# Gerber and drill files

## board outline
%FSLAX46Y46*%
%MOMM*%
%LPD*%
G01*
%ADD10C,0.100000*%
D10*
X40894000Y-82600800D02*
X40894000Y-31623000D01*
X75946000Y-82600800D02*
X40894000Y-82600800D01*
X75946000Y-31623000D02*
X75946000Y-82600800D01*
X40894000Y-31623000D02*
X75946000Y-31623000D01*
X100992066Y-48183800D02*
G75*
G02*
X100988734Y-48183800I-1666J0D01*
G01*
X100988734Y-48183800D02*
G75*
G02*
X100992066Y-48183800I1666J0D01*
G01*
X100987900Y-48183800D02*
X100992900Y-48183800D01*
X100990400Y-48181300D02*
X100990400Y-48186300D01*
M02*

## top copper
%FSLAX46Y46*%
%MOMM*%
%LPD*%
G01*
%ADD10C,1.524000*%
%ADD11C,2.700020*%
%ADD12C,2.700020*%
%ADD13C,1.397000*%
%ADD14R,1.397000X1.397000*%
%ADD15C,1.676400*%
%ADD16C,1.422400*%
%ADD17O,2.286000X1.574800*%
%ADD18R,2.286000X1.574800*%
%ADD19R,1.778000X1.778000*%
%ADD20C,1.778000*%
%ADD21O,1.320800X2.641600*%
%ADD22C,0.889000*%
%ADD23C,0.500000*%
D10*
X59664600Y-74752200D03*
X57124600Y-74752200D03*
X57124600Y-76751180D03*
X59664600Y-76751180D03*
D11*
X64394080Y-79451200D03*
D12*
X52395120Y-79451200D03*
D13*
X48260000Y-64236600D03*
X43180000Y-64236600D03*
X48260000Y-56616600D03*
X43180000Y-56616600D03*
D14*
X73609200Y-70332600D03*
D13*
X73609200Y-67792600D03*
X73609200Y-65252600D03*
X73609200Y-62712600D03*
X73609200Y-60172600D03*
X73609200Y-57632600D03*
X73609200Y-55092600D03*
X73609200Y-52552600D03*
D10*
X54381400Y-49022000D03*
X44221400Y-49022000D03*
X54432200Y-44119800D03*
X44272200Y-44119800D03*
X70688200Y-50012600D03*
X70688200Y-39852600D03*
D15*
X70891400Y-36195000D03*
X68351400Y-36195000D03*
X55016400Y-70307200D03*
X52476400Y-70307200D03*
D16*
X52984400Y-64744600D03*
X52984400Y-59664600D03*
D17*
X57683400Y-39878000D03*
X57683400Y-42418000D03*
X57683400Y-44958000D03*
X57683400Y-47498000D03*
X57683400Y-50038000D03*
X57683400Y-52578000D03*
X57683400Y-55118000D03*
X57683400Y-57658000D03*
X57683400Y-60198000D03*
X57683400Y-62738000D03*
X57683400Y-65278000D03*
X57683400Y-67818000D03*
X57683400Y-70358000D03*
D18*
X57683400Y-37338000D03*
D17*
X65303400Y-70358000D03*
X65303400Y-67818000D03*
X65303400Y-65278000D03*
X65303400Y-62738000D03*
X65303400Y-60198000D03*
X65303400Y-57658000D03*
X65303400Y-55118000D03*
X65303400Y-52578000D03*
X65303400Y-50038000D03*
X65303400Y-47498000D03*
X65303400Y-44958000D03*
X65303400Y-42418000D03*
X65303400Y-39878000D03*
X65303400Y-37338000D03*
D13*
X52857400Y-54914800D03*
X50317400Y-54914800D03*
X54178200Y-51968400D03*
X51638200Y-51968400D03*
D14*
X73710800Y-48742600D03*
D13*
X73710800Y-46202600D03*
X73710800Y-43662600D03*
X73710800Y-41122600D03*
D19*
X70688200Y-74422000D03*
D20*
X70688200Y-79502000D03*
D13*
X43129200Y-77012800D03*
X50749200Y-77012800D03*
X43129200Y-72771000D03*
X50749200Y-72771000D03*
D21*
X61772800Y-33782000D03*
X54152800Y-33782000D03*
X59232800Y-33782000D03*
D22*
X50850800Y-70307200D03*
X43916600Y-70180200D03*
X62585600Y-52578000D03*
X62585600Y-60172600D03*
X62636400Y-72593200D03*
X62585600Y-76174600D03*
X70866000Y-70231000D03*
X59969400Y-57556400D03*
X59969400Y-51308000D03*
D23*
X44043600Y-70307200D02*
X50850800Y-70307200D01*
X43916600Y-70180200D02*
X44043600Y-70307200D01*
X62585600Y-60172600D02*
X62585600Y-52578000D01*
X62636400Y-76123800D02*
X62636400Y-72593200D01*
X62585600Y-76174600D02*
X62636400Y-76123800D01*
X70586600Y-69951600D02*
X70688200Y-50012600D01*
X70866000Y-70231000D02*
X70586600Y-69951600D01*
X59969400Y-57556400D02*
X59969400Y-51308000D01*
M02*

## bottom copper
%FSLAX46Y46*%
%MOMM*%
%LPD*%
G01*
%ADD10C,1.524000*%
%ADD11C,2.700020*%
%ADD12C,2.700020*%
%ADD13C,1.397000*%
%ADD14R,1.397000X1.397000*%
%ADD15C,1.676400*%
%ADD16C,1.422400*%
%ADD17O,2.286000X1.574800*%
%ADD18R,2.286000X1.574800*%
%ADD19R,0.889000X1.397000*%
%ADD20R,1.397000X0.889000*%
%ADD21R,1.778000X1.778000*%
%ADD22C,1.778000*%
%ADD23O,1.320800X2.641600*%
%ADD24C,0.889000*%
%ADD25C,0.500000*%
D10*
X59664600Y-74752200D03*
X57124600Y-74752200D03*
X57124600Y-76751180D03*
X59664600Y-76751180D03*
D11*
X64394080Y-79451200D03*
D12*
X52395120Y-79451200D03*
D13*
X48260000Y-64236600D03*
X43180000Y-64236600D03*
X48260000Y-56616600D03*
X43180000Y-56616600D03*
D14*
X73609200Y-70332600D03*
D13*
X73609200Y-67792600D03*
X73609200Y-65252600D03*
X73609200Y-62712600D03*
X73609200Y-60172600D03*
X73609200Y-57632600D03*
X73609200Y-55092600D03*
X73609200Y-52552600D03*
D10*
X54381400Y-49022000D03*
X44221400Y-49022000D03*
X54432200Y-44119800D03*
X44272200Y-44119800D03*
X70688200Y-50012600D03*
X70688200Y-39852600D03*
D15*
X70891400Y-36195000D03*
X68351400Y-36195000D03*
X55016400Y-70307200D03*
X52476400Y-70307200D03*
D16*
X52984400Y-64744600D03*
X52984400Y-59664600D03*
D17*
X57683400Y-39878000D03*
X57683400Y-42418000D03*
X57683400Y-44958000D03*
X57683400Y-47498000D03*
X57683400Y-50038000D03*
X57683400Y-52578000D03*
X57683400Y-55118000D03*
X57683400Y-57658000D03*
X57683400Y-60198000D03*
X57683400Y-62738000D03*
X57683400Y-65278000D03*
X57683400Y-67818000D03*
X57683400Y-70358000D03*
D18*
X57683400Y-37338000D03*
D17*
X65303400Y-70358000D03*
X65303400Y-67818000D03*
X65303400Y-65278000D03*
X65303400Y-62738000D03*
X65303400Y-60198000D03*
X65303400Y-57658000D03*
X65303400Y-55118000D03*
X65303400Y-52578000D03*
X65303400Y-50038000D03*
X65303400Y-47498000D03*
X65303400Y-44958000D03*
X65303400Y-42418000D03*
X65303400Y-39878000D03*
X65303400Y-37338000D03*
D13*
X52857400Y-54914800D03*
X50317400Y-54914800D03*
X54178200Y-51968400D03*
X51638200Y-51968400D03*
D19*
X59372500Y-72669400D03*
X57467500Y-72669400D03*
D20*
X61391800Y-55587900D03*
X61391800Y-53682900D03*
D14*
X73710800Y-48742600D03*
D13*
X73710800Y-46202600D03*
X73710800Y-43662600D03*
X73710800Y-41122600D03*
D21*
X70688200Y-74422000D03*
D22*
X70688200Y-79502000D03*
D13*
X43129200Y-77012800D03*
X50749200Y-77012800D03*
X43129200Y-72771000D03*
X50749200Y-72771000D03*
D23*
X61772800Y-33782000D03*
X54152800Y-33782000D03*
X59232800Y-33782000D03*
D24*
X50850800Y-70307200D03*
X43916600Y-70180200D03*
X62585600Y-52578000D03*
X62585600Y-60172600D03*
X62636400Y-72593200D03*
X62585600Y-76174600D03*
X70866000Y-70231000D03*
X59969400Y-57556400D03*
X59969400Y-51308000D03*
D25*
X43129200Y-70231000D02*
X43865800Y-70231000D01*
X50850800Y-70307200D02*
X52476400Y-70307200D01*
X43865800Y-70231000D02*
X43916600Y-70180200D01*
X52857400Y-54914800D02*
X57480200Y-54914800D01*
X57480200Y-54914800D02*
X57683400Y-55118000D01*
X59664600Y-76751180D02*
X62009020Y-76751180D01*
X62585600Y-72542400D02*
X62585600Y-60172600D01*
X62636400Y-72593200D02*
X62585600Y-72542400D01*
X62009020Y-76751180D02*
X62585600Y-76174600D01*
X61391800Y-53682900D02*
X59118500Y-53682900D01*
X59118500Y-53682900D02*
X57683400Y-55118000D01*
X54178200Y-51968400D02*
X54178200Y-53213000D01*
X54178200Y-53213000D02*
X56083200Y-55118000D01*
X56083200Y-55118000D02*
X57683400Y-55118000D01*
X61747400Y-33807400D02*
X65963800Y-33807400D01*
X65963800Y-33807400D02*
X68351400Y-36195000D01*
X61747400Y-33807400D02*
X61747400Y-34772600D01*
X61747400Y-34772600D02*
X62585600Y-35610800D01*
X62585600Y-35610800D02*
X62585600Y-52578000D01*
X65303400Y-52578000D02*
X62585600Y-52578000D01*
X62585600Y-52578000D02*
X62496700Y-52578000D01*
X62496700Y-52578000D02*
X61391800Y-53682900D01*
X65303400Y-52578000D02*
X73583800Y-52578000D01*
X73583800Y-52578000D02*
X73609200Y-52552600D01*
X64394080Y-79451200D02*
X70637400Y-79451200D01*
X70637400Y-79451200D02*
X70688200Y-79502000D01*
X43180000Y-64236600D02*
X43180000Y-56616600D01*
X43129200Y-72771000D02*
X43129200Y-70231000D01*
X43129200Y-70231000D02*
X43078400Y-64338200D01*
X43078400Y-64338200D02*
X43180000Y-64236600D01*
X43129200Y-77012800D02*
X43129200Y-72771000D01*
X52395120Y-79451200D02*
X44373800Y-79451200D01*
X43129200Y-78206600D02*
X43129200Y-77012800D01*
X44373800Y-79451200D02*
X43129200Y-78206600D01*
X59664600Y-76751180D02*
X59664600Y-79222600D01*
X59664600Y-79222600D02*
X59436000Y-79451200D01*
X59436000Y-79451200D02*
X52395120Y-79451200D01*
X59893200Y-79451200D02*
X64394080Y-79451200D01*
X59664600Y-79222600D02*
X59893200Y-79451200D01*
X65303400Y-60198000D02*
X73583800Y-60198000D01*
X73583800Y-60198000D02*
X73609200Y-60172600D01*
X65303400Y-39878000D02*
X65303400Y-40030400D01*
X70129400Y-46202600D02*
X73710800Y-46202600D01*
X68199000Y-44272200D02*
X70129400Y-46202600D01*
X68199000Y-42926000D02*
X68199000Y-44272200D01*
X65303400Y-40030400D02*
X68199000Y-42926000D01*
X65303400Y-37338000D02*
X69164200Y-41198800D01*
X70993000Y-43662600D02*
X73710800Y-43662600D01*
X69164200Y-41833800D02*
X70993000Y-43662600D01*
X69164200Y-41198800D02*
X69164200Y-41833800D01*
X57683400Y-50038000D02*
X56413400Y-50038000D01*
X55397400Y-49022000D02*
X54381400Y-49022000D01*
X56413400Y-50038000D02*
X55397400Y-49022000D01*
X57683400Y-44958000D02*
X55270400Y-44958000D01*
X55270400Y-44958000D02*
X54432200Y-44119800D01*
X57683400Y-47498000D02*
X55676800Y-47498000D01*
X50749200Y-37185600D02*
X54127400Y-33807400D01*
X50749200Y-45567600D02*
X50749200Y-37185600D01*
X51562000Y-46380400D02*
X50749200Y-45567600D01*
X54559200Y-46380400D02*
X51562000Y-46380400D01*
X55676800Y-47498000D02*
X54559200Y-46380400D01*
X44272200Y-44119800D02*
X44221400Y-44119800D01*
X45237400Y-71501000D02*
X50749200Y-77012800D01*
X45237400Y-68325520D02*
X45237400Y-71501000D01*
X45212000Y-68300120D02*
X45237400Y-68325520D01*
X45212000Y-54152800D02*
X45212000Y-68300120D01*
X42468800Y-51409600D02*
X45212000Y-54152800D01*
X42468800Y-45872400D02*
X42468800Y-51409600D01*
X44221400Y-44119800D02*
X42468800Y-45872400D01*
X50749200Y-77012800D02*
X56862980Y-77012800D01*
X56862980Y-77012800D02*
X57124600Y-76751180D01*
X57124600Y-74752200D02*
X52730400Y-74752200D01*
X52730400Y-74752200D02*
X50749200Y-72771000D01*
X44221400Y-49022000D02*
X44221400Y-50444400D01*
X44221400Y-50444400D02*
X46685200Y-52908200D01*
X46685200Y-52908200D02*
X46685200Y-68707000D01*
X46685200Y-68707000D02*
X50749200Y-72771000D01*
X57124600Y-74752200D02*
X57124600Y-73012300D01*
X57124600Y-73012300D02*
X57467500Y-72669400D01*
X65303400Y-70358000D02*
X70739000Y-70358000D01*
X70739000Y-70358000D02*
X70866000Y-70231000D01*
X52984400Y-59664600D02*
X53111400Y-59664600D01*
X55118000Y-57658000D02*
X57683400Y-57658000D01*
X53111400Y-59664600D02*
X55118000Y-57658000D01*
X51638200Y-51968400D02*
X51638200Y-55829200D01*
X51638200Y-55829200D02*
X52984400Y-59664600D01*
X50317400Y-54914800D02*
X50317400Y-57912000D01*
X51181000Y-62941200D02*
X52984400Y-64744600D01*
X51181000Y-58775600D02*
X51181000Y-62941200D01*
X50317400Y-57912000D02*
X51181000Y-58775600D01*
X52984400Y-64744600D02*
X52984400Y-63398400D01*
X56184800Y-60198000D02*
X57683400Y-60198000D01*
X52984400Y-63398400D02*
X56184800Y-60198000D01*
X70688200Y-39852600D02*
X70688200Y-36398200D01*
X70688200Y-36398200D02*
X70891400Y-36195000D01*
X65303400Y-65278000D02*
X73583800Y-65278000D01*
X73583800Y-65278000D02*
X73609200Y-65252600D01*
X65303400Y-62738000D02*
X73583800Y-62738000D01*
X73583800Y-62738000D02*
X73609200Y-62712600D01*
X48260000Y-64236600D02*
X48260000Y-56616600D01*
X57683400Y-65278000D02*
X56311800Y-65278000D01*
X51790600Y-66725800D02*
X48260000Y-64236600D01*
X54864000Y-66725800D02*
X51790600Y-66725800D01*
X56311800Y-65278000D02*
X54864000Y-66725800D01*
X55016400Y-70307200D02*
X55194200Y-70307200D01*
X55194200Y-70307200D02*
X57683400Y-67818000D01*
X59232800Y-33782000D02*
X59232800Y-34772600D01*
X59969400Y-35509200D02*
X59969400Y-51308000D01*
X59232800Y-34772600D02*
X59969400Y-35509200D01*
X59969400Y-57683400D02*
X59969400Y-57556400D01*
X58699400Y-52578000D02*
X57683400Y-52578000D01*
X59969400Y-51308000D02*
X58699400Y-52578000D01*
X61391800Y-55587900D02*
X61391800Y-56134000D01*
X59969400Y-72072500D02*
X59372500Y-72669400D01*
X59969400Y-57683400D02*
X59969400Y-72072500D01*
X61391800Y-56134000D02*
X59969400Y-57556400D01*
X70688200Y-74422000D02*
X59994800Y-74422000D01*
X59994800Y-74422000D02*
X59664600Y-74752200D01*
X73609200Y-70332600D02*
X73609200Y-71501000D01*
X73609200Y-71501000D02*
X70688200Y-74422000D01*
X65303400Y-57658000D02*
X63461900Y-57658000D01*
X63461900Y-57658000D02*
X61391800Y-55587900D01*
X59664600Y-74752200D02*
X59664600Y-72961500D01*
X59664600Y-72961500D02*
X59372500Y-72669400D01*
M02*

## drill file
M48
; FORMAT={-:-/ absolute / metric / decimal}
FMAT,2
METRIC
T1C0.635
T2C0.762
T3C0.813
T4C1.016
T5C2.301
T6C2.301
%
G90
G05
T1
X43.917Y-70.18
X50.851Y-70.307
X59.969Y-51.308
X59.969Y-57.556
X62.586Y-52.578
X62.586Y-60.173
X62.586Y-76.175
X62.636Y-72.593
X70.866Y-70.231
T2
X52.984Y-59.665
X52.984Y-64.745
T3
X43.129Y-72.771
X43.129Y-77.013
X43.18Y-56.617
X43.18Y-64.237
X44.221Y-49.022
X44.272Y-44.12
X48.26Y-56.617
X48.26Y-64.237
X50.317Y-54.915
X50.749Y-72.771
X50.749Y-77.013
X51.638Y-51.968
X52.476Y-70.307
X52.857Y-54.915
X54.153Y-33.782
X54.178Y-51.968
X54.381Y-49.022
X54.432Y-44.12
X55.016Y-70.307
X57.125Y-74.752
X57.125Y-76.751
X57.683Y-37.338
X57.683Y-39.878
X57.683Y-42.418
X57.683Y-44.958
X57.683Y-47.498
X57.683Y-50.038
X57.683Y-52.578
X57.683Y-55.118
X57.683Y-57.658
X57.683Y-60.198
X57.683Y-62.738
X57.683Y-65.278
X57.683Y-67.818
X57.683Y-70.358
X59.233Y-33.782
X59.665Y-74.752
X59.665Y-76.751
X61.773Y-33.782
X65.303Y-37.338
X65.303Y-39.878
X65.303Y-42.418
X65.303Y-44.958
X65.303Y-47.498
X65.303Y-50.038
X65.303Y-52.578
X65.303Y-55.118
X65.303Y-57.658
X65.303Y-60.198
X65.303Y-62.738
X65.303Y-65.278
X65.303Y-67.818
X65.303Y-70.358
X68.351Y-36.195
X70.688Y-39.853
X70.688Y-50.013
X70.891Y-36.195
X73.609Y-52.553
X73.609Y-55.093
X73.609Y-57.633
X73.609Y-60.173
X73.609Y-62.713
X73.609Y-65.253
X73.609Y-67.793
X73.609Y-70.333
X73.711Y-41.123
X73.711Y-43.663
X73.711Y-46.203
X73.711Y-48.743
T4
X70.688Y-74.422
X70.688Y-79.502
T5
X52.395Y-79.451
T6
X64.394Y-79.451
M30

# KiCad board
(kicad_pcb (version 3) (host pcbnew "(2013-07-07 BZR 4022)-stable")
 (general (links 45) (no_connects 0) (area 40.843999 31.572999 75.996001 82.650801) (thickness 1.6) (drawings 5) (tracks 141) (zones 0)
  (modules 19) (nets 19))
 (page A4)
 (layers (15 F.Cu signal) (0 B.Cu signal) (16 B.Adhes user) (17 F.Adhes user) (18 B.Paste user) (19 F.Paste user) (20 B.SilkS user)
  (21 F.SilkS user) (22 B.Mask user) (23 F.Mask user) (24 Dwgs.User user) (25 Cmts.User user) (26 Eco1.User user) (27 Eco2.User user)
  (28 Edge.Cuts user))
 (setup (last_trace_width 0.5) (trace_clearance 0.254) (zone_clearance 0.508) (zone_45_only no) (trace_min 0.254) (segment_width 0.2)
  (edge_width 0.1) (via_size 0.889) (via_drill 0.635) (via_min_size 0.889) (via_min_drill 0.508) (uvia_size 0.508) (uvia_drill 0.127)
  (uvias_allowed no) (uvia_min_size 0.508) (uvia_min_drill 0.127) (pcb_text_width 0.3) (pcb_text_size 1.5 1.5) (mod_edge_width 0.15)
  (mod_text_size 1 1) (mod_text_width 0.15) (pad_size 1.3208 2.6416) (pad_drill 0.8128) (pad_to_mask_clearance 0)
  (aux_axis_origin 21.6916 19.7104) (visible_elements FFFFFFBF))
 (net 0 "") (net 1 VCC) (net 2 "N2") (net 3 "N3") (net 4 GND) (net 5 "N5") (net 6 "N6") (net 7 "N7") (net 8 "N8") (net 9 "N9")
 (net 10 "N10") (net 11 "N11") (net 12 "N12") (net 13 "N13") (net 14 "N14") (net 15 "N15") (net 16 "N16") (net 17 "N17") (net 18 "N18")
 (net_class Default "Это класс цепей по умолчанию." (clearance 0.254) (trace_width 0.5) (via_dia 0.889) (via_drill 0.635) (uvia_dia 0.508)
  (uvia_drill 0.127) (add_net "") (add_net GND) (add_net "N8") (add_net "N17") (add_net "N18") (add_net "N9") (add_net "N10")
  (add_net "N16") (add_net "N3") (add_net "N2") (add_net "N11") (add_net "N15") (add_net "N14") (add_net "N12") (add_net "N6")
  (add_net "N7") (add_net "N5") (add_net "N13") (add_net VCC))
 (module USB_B (layer F.Cu) (at 58.3946 79.4512)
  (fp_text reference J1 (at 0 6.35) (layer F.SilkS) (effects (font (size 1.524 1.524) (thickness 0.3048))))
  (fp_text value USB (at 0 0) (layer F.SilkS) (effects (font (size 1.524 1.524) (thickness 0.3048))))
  (pad 1 thru_hole circle (at 1.27 -4.699) (size 1.524 1.524) (drill 0.8128) (layers *.Cu *.Mask F.SilkS) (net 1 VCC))
  (pad 2 thru_hole circle (at -1.27 -4.699) (size 1.524 1.524) (drill 0.8128) (layers *.Cu *.Mask F.SilkS) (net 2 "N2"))
  (pad 3 thru_hole circle (at -1.27 -2.70002) (size 1.524 1.524) (drill 0.8128) (layers *.Cu *.Mask F.SilkS) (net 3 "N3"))
  (pad 4 thru_hole circle (at 1.27 -2.70002) (size 1.524 1.524) (drill 0.8128) (layers *.Cu *.Mask F.SilkS) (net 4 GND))
  (pad 5 np_thru_hole circle (at 5.99948 0) (size 2.70002 2.70002) (drill 2.30124) (layers *.Cu *.SilkS *.Mask) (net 4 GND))
  (pad 6 thru_hole circle (at -5.99948 0) (size 2.70002 2.70002) (drill 2.30124) (layers *.Cu *.Mask F.SilkS) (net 4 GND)))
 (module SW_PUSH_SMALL (layer F.Cu) (at 45.72 60.4266 270)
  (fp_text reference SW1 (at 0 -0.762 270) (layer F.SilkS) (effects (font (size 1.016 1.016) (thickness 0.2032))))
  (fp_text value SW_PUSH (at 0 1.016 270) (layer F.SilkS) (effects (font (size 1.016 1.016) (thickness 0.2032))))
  (pad 1 thru_hole circle (at 3.81 -2.54 270) (size 1.397 1.397) (drill 0.8128) (layers *.Cu *.Mask F.SilkS) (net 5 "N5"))
  (pad 2 thru_hole circle (at 3.81 2.54 270) (size 1.397 1.397) (drill 0.8128) (layers *.Cu *.Mask F.SilkS) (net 4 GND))
  (pad 1 thru_hole circle (at -3.81 -2.54 270) (size 1.397 1.397) (drill 0.8128) (layers *.Cu *.Mask F.SilkS) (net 5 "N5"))
  (pad 2 thru_hole circle (at -3.81 2.54 270) (size 1.397 1.397) (drill 0.8128) (layers *.Cu *.Mask F.SilkS) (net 4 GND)))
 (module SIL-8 (layer F.Cu) (at 73.6092 61.4426 90)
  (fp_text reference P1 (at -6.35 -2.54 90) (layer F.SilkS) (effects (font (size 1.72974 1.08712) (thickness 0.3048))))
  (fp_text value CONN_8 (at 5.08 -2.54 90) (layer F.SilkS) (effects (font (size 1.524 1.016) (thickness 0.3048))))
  (pad 1 thru_hole rect (at -8.89 0 90) (size 1.397 1.397) (drill 0.8128) (layers *.Cu *.Mask F.SilkS) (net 1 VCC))
  (pad 2 thru_hole circle (at -6.35 0 90) (size 1.397 1.397) (drill 0.8128) (layers *.Cu *.Mask F.SilkS))
  (pad 3 thru_hole circle (at -3.81 0 90) (size 1.397 1.397) (drill 0.8128) (layers *.Cu *.Mask F.SilkS) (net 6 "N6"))
  (pad 4 thru_hole circle (at -1.27 0 90) (size 1.397 1.397) (drill 0.8128) (layers *.Cu *.Mask F.SilkS) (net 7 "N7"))
  (pad 5 thru_hole circle (at 1.27 0 90) (size 1.397 1.397) (drill 0.8128) (layers *.Cu *.Mask F.SilkS) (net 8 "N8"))
  (pad 6 thru_hole circle (at 3.81 0 90) (size 1.397 1.397) (drill 0.8128) (layers *.Cu *.Mask F.SilkS))
  (pad 7 thru_hole circle (at 6.35 0 90) (size 1.397 1.397) (drill 0.8128) (layers *.Cu *.Mask F.SilkS))
  (pad 8 thru_hole circle (at 8.89 0 90) (size 1.397 1.397) (drill 0.8128) (layers *.Cu *.Mask F.SilkS) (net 4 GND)))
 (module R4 (layer F.Cu) (at 49.3014 49.022 180) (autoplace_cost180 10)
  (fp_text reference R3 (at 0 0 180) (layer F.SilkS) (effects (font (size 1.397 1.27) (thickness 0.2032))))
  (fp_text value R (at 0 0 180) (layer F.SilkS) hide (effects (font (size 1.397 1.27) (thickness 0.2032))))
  (pad 1 thru_hole circle (at -5.08 0 180) (size 1.524 1.524) (drill 0.8128) (layers *.Cu *.Mask F.SilkS) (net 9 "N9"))
  (pad 2 thru_hole circle (at 5.08 0 180) (size 1.524 1.524) (drill 0.8128) (layers *.Cu *.Mask F.SilkS) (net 2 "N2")))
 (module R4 (layer F.Cu) (at 49.3522 44.1198 180) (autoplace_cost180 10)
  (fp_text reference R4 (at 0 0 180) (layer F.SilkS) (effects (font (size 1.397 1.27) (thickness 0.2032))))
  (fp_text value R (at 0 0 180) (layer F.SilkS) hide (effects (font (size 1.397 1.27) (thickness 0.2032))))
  (pad 1 thru_hole circle (at -5.08 0 180) (size 1.524 1.524) (drill 0.8128) (layers *.Cu *.Mask F.SilkS) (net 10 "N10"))
  (pad 2 thru_hole circle (at 5.08 0 180) (size 1.524 1.524) (drill 0.8128) (layers *.Cu *.Mask F.SilkS) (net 3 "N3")))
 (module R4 (layer F.Cu) (at 70.6882 44.9326 90) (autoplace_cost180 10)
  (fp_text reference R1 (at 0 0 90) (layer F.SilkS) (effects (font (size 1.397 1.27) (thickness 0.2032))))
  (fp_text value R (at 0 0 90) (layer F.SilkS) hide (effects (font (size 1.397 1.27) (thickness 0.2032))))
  (pad 1 thru_hole circle (at -5.08 0 90) (size 1.524 1.524) (drill 0.8128) (layers *.Cu *.Mask F.SilkS) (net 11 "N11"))
  (pad 2 thru_hole circle (at 5.08 0 90) (size 1.524 1.524) (drill 0.8128) (layers *.Cu *.Mask F.SilkS) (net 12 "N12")))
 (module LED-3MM (layer F.Cu) (at 69.6214 36.195 180)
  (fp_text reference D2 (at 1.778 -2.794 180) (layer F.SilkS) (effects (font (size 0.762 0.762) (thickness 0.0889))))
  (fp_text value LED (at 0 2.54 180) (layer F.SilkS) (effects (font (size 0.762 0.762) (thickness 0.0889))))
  (pad 1 thru_hole circle (at -1.27 0 180) (size 1.6764 1.6764) (drill 0.8128) (layers *.Cu *.Mask F.SilkS) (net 12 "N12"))
  (pad 2 thru_hole circle (at 1.27 0 180) (size 1.6764 1.6764) (drill 0.8128) (layers *.Cu *.Mask F.SilkS) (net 4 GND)))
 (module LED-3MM (layer F.Cu) (at 53.7464 70.3072 180)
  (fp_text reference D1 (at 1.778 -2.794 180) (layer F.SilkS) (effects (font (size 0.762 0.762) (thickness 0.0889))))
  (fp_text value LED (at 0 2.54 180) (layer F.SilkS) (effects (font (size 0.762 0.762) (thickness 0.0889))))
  (pad 1 thru_hole circle (at -1.27 0 180) (size 1.6764 1.6764) (drill 0.8128) (layers *.Cu *.Mask F.SilkS) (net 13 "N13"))
  (pad 2 thru_hole circle (at 1.27 0 180) (size 1.6764 1.6764) (drill 0.8128) (layers *.Cu *.Mask F.SilkS) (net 4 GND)))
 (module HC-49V (layer F.Cu) (at 52.9844 62.2046 90) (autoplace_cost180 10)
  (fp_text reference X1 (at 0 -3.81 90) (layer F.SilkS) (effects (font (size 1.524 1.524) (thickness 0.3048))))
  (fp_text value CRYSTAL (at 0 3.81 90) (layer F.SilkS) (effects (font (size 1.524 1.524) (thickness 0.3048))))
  (pad 1 thru_hole circle (at -2.54 0 90) (size 1.4224 1.4224) (drill 0.762) (layers *.Cu *.Mask F.SilkS) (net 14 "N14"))
  (pad 2 thru_hole circle (at 2.54 0 90) (size 1.4224 1.4224) (drill 0.762) (layers *.Cu *.Mask F.SilkS) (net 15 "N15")))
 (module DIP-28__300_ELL (layer F.Cu) (at 61.4934 53.848 270)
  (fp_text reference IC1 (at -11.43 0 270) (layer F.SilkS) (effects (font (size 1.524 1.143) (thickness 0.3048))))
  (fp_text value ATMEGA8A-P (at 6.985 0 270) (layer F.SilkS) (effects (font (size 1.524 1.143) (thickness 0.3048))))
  (pad 2 thru_hole oval (at -13.97 3.81 270) (size 1.5748 2.286) (drill 0.8128) (layers *.Cu *.Mask F.SilkS))
  (pad 3 thru_hole oval (at -11.43 3.81 270) (size 1.5748 2.286) (drill 0.8128) (layers *.Cu *.Mask F.SilkS))
  (pad 4 thru_hole oval (at -8.89 3.81 270) (size 1.5748 2.286) (drill 0.8128) (layers *.Cu *.Mask F.SilkS) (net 10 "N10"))
  (pad 5 thru_hole oval (at -6.35 3.81 270) (size 1.5748 2.286) (drill 0.8128) (layers *.Cu *.Mask F.SilkS) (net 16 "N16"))
  (pad 6 thru_hole oval (at -3.81 3.81 270) (size 1.5748 2.286) (drill 0.8128) (layers *.Cu *.Mask F.SilkS) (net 9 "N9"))
  (pad 7 thru_hole oval (at -1.27 3.81 270) (size 1.5748 2.286) (drill 0.8128) (layers *.Cu *.Mask F.SilkS) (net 1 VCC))
  (pad 8 thru_hole oval (at 1.27 3.81 270) (size 1.5748 2.286) (drill 0.8128) (layers *.Cu *.Mask F.SilkS) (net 4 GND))
  (pad 9 thru_hole oval (at 3.81 3.81 270) (size 1.5748 2.286) (drill 0.8128) (layers *.Cu *.Mask F.SilkS) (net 15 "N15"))
  (pad 10 thru_hole oval (at 6.35 3.81 270) (size 1.5748 2.286) (drill 0.8128) (layers *.Cu *.Mask F.SilkS) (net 14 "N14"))
  (pad 11 thru_hole oval (at 8.89 3.81 270) (size 1.5748 2.286) (drill 0.8128) (layers *.Cu *.Mask F.SilkS))
  (pad 12 thru_hole oval (at 11.43 3.81 270) (size 1.5748 2.286) (drill 0.8128) (layers *.Cu *.Mask F.SilkS) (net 5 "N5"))
  (pad 13 thru_hole oval (at 13.97 3.81 270) (size 1.5748 2.286) (drill 0.8128) (layers *.Cu *.Mask F.SilkS) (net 13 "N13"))
  (pad 14 thru_hole oval (at 16.51 3.81 270) (size 1.5748 2.286) (drill 0.8128) (layers *.Cu *.Mask F.SilkS))
  (pad 1 thru_hole rect (at -16.51 3.81 270) (size 1.5748 2.286) (drill 0.8128) (layers *.Cu *.Mask F.SilkS))
  (pad 15 thru_hole oval (at 16.51 -3.81 270) (size 1.5748 2.286) (drill 0.8128) (layers *.Cu *.Mask F.SilkS) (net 11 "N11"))
  (pad 16 thru_hole oval (at 13.97 -3.81 270) (size 1.5748 2.286) (drill 0.8128) (layers *.Cu *.Mask F.SilkS))
  (pad 17 thru_hole oval (at 11.43 -3.81 270) (size 1.5748 2.286) (drill 0.8128) (layers *.Cu *.Mask F.SilkS) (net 6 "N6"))
  (pad 18 thru_hole oval (at 8.89 -3.81 270) (size 1.5748 2.286) (drill 0.8128) (layers *.Cu *.Mask F.SilkS) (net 7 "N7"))
  (pad 19 thru_hole oval (at 6.35 -3.81 270) (size 1.5748 2.286) (drill 0.8128) (layers *.Cu *.Mask F.SilkS) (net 8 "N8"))
  (pad 20 thru_hole oval (at 3.81 -3.81 270) (size 1.5748 2.286) (drill 0.8128) (layers *.Cu *.Mask F.SilkS) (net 1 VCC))
  (pad 21 thru_hole oval (at 1.27 -3.81 270) (size 1.5748 2.286) (drill 0.8128) (layers *.Cu *.Mask F.SilkS))
  (pad 22 thru_hole oval (at -1.27 -3.81 270) (size 1.5748 2.286) (drill 0.8128) (layers *.Cu *.Mask F.SilkS) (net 4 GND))
  (pad 23 thru_hole oval (at -3.81 -3.81 270) (size 1.5748 2.286) (drill 0.8128) (layers *.Cu *.Mask F.SilkS))
  (pad 24 thru_hole oval (at -6.35 -3.81 270) (size 1.5748 2.286) (drill 0.8128) (layers *.Cu *.Mask F.SilkS))
  (pad 25 thru_hole oval (at -8.89 -3.81 270) (size 1.5748 2.286) (drill 0.8128) (layers *.Cu *.Mask F.SilkS))
  (pad 26 thru_hole oval (at -11.43 -3.81 270) (size 1.5748 2.286) (drill 0.8128) (layers *.Cu *.Mask F.SilkS))
  (pad 27 thru_hole oval (at -13.97 -3.81 270) (size 1.5748 2.286) (drill 0.8128) (layers *.Cu *.Mask F.SilkS) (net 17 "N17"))
  (pad 28 thru_hole oval (at -16.51 -3.81 270) (size 1.5748 2.286) (drill 0.8128) (layers *.Cu *.Mask F.SilkS) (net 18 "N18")))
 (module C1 (layer F.Cu) (at 51.5874 54.9148 180)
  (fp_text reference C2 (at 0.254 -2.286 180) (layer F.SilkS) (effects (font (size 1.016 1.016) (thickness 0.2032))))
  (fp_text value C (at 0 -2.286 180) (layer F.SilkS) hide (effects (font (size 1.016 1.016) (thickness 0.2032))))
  (pad 1 thru_hole circle (at -1.27 0 180) (size 1.397 1.397) (drill 0.8128) (layers *.Cu *.Mask F.SilkS) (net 4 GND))
  (pad 2 thru_hole circle (at 1.27 0 180) (size 1.397 1.397) (drill 0.8128) (layers *.Cu *.Mask F.SilkS) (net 14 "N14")))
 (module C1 (layer F.Cu) (at 52.9082 51.9684 180)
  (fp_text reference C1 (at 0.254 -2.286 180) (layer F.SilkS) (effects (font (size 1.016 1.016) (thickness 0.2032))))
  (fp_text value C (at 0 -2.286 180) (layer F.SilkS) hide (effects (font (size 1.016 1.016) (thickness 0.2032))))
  (pad 1 thru_hole circle (at -1.27 0 180) (size 1.397 1.397) (drill 0.8128) (layers *.Cu *.Mask F.SilkS) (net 4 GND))
  (pad 2 thru_hole circle (at 1.27 0 180) (size 1.397 1.397) (drill 0.8128) (layers *.Cu *.Mask F.SilkS) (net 15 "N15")))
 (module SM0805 (layer B.Cu) (at 58.42 72.6694 180)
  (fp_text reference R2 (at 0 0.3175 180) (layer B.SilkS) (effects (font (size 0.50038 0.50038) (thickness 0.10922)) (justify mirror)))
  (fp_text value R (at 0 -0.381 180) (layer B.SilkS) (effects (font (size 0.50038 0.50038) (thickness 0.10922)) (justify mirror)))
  (pad 1 smd rect (at -0.9525 0 180) (size 0.889 1.397) (layers B.Cu B.Paste B.Mask) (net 1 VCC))
  (pad 2 smd rect (at 0.9525 0 180) (size 0.889 1.397) (layers B.Cu B.Paste B.Mask) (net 2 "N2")))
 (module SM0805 (layer B.Cu) (at 61.3918 54.6354 90)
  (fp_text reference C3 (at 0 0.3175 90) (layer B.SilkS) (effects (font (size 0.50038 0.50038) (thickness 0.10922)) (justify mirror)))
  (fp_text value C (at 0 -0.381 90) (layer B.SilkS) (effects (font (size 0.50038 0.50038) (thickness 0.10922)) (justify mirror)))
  (pad 1 smd rect (at -0.9525 0 90) (size 0.889 1.397) (layers B.Cu B.Paste B.Mask) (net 1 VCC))
  (pad 2 smd rect (at 0.9525 0 90) (size 0.889 1.397) (layers B.Cu B.Paste B.Mask) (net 4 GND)))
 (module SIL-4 (layer F.Cu) (at 73.7108 44.9326 90)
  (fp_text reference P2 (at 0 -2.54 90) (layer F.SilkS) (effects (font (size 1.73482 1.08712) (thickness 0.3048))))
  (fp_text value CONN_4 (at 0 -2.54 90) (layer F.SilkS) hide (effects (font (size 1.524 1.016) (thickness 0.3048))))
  (pad 1 thru_hole rect (at -3.81 0 90) (size 1.397 1.397) (drill 0.8128) (layers *.Cu *.Mask F.SilkS))
  (pad 2 thru_hole circle (at -1.27 0 90) (size 1.397 1.397) (drill 0.8128) (layers *.Cu *.Mask F.SilkS) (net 17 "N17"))
  (pad 3 thru_hole circle (at 1.27 0 90) (size 1.397 1.397) (drill 0.8128) (layers *.Cu *.Mask F.SilkS) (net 18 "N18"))
  (pad 4 thru_hole circle (at 3.81 0 90) (size 1.397 1.397) (drill 0.8128) (layers *.Cu *.Mask F.SilkS)))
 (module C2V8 (layer F.Cu) (at 70.6882 76.962 270)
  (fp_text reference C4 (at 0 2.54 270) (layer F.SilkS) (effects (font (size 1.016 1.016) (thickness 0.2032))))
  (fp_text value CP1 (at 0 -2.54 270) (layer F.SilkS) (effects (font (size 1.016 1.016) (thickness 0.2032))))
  (pad 1 thru_hole rect (at -2.54 0 270) (size 1.778 1.778) (drill 1.016) (layers *.Cu *.Mask F.SilkS) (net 1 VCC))
  (pad 2 thru_hole circle (at 2.54 0 270) (size 1.778 1.778) (drill 1.016) (layers *.Cu *.Mask F.SilkS) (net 4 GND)))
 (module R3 (layer F.Cu) (at 46.9392 77.0128) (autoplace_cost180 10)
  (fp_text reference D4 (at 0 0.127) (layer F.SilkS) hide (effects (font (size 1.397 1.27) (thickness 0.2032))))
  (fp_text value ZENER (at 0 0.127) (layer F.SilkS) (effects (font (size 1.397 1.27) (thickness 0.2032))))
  (pad 1 thru_hole circle (at -3.81 0) (size 1.397 1.397) (drill 0.8128) (layers *.Cu *.Mask F.SilkS) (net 4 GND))
  (pad 2 thru_hole circle (at 3.81 0) (size 1.397 1.397) (drill 0.8128) (layers *.Cu *.Mask F.SilkS) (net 3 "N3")))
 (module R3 (layer F.Cu) (at 46.9392 72.771) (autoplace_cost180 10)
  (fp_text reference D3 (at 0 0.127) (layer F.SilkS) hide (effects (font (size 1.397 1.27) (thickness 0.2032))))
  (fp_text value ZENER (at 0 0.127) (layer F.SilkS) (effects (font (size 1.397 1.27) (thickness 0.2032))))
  (pad 1 thru_hole circle (at -3.81 0) (size 1.397 1.397) (drill 0.8128) (layers *.Cu *.Mask F.SilkS) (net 4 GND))
  (pad 2 thru_hole circle (at 3.81 0) (size 1.397 1.397) (drill 0.8128) (layers *.Cu *.Mask F.SilkS) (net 2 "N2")))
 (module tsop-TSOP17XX (layer F.Cu) (at 57.9628 33.782 180)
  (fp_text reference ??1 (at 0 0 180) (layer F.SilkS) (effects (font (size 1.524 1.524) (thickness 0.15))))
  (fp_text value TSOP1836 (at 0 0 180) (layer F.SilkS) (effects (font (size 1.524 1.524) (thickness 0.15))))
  (pad GND thru_hole oval (at -3.81 0 180) (size 1.3208 2.6416) (drill 0.8128) (layers *.Cu F.Paste F.SilkS F.Mask) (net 4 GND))
  (pad OUT thru_hole oval (at 3.81 0 180) (size 1.3208 2.6416) (drill 0.8128) (layers *.Cu F.Paste F.SilkS F.Mask) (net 16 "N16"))
  (pad VCC thru_hole oval (at -1.27 0 180) (size 1.3208 2.6416) (drill 0.8128) (layers *.Cu F.Paste F.SilkS F.Mask) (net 1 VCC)))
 (gr_line (start 40.894 82.6008) (end 40.894 31.623) (angle 90) (layer Edge.Cuts) (width 0.1))
 (gr_line (start 75.946 82.6008) (end 40.894 82.6008) (angle 90) (layer Edge.Cuts) (width 0.1))
 (gr_line (start 75.946 31.623) (end 75.946 82.6008) (angle 90) (layer Edge.Cuts) (width 0.1))
 (gr_line (start 40.894 31.623) (end 75.946 31.623) (angle 90) (layer Edge.Cuts) (width 0.1))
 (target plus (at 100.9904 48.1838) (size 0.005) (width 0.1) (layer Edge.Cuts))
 (segment (start 43.1292 70.231) (end 43.8658 70.231) (width 0.5) (layer B.Cu) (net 4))
 (segment (start 50.8508 70.3072) (end 52.4764 70.3072) (width 0.5) (layer B.Cu) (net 4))
 (via (at 50.8508 70.3072) (size 0.889) (layers F.Cu B.Cu) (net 4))
 (segment (start 44.0436 70.3072) (end 50.8508 70.3072) (width 0.5) (layer F.Cu) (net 4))
 (segment (start 43.9166 70.1802) (end 44.0436 70.3072) (width 0.5) (layer F.Cu) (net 4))
 (via (at 43.9166 70.1802) (size 0.889) (layers F.Cu B.Cu) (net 4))
 (segment (start 43.8658 70.231) (end 43.9166 70.1802) (width 0.5) (layer B.Cu) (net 4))
 (segment (start 52.8574 54.9148) (end 57.4802 54.9148) (width 0.5) (layer B.Cu) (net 4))
 (segment (start 57.4802 54.9148) (end 57.6834 55.118) (width 0.5) (layer B.Cu) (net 4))
 (segment (start 59.6646 76.75118) (end 62.00902 76.75118) (width 0.5) (layer B.Cu) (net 4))
 (via (at 62.5856 52.578) (size 0.889) (layers F.Cu B.Cu) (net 4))
 (segment (start 62.5856 60.1726) (end 62.5856 52.578) (width 0.5) (layer F.Cu) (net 4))
 (via (at 62.5856 60.1726) (size 0.889) (layers F.Cu B.Cu) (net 4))
 (segment (start 62.5856 72.5424) (end 62.5856 60.1726) (width 0.5) (layer B.Cu) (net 4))
 (segment (start 62.6364 72.5932) (end 62.5856 72.5424) (width 0.5) (layer B.Cu) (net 4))
 (via (at 62.6364 72.5932) (size 0.889) (layers F.Cu B.Cu) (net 4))
 (segment (start 62.6364 76.1238) (end 62.6364 72.5932) (width 0.5) (layer F.Cu) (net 4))
 (segment (start 62.5856 76.1746) (end 62.6364 76.1238) (width 0.5) (layer F.Cu) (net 4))
 (via (at 62.5856 76.1746) (size 0.889) (layers F.Cu B.Cu) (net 4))
 (segment (start 62.00902 76.75118) (end 62.5856 76.1746) (width 0.5) (layer B.Cu) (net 4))
 (segment (start 61.3918 53.6829) (end 59.1185 53.6829) (width 0.5) (layer B.Cu) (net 4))
 (segment (start 59.1185 53.6829) (end 57.6834 55.118) (width 0.5) (layer B.Cu) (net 4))
 (segment (start 54.1782 51.9684) (end 54.1782 53.213) (width 0.5) (layer B.Cu) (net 4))
 (segment (start 54.1782 53.213) (end 56.0832 55.118) (width 0.5) (layer B.Cu) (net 4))
 (segment (start 56.0832 55.118) (end 57.6834 55.118) (width 0.5) (layer B.Cu) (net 4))
 (segment (start 61.7474 33.8074) (end 65.9638 33.8074) (width 0.5) (layer B.Cu) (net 4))
 (segment (start 65.9638 33.8074) (end 68.3514 36.195) (width 0.5) (layer B.Cu) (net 4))
 (segment (start 61.7474 33.8074) (end 61.7474 34.7726) (width 0.5) (layer B.Cu) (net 4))
 (segment (start 61.7474 34.7726) (end 62.5856 35.6108) (width 0.5) (layer B.Cu) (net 4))
 (segment (start 62.5856 35.6108) (end 62.5856 52.578) (width 0.5) (layer B.Cu) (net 4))
 (segment (start 65.3034 52.578) (end 62.5856 52.578) (width 0.5) (layer B.Cu) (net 4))
 (segment (start 62.5856 52.578) (end 62.4967 52.578) (width 0.5) (layer B.Cu) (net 4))
 (segment (start 62.4967 52.578) (end 61.3918 53.6829) (width 0.5) (layer B.Cu) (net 4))
 (segment (start 65.3034 52.578) (end 73.5838 52.578) (width 0.5) (layer B.Cu) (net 4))
 (segment (start 73.5838 52.578) (end 73.6092 52.5526) (width 0.5) (layer B.Cu) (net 4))
 (segment (start 64.39408 79.4512) (end 70.6374 79.4512) (width 0.5) (layer B.Cu) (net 4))
 (segment (start 70.6374 79.4512) (end 70.6882 79.502) (width 0.5) (layer B.Cu) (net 4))
 (segment (start 43.18 64.2366) (end 43.18 56.6166) (width 0.5) (layer B.Cu) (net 4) (status 30))
 (segment (start 43.1292 72.771) (end 43.1292 70.231) (width 0.5) (layer B.Cu) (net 4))
 (segment (start 43.1292 70.231) (end 43.0784 64.3382) (width 0.5) (layer B.Cu) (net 4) (status 20))
 (segment (start 43.0784 64.3382) (end 43.18 64.2366) (width 0.5) (layer B.Cu) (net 4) (status 30))
 (segment (start 43.1292 77.0128) (end 43.1292 72.771) (width 0.5) (layer B.Cu) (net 4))
 (segment (start 52.39512 79.4512) (end 44.3738 79.4512) (width 0.5) (layer B.Cu) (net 4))
 (segment (start 43.1292 78.2066) (end 43.1292 77.0128) (width 0.5) (layer B.Cu) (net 4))
 (segment (start 44.3738 79.4512) (end 43.1292 78.2066) (width 0.5) (layer B.Cu) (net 4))
 (segment (start 59.6646 76.75118) (end 59.6646 79.2226) (width 0.5) (layer B.Cu) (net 4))
 (segment (start 59.6646 79.2226) (end 59.436 79.4512) (width 0.5) (layer B.Cu) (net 4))
 (segment (start 59.436 79.4512) (end 52.39512 79.4512) (width 0.5) (layer B.Cu) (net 4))
 (segment (start 59.8932 79.4512) (end 64.39408 79.4512) (width 0.5) (layer B.Cu) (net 4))
 (segment (start 59.6646 79.2226) (end 59.8932 79.4512) (width 0.5) (layer B.Cu) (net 4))
 (segment (start 65.3034 60.198) (end 73.5838 60.198) (width 0.5) (layer B.Cu) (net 8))
 (segment (start 73.5838 60.198) (end 73.6092 60.1726) (width 0.5) (layer B.Cu) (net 8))
 (segment (start 65.3034 39.878) (end 65.3034 40.0304) (width 0.5) (layer B.Cu) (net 17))
 (segment (start 70.1294 46.2026) (end 73.7108 46.2026) (width 0.5) (layer B.Cu) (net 17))
 (segment (start 68.199 44.2722) (end 70.1294 46.2026) (width 0.5) (layer B.Cu) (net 17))
 (segment (start 68.199 42.926) (end 68.199 44.2722) (width 0.5) (layer B.Cu) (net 17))
 (segment (start 65.3034 40.0304) (end 68.199 42.926) (width 0.5) (layer B.Cu) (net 17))
 (segment (start 65.3034 37.338) (end 69.1642 41.1988) (width 0.5) (layer B.Cu) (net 18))
 (segment (start 70.993 43.6626) (end 73.7108 43.6626) (width 0.5) (layer B.Cu) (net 18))
 (segment (start 69.1642 41.8338) (end 70.993 43.6626) (width 0.5) (layer B.Cu) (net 18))
 (segment (start 69.1642 41.1988) (end 69.1642 41.8338) (width 0.5) (layer B.Cu) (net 18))
 (segment (start 57.6834 50.038) (end 56.4134 50.038) (width 0.5) (layer B.Cu) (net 9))
 (segment (start 55.3974 49.022) (end 54.3814 49.022) (width 0.5) (layer B.Cu) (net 9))
 (segment (start 56.4134 50.038) (end 55.3974 49.022) (width 0.5) (layer B.Cu) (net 9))
 (segment (start 57.6834 44.958) (end 55.2704 44.958) (width 0.5) (layer B.Cu) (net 10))
 (segment (start 55.2704 44.958) (end 54.4322 44.1198) (width 0.5) (layer B.Cu) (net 10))
 (segment (start 57.6834 47.498) (end 55.6768 47.498) (width 0.5) (layer B.Cu) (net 16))
 (segment (start 50.7492 37.1856) (end 54.1274 33.8074) (width 0.5) (layer B.Cu) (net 16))
 (segment (start 50.7492 45.5676) (end 50.7492 37.1856) (width 0.5) (layer B.Cu) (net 16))
 (segment (start 51.562 46.3804) (end 50.7492 45.5676) (width 0.5) (layer B.Cu) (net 16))
 (segment (start 54.5592 46.3804) (end 51.562 46.3804) (width 0.5) (layer B.Cu) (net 16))
 (segment (start 55.6768 47.498) (end 54.5592 46.3804) (width 0.5) (layer B.Cu) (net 16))
 (segment (start 44.2722 44.1198) (end 44.2214 44.1198) (width 0.5) (layer B.Cu) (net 3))
 (segment (start 45.2374 71.501) (end 50.7492 77.0128) (width 0.5) (layer B.Cu) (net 3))
 (segment (start 45.2374 68.32552) (end 45.2374 71.501) (width 0.5) (layer B.Cu) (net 3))
 (segment (start 45.212 68.30012) (end 45.2374 68.32552) (width 0.5) (layer B.Cu) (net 3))
 (segment (start 45.212 54.1528) (end 45.212 68.30012) (width 0.5) (layer B.Cu) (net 3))
 (segment (start 42.4688 51.4096) (end 45.212 54.1528) (width 0.5) (layer B.Cu) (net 3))
 (segment (start 42.4688 45.8724) (end 42.4688 51.4096) (width 0.5) (layer B.Cu) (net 3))
 (segment (start 44.2214 44.1198) (end 42.4688 45.8724) (width 0.5) (layer B.Cu) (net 3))
 (segment (start 50.7492 77.0128) (end 56.86298 77.0128) (width 0.5) (layer B.Cu) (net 3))
 (segment (start 56.86298 77.0128) (end 57.1246 76.75118) (width 0.5) (layer B.Cu) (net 3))
 (segment (start 57.1246 74.7522) (end 52.7304 74.7522) (width 0.5) (layer B.Cu) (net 2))
 (segment (start 52.7304 74.7522) (end 50.7492 72.771) (width 0.5) (layer B.Cu) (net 2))
 (segment (start 44.2214 49.022) (end 44.2214 50.4444) (width 0.5) (layer B.Cu) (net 2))
 (segment (start 44.2214 50.4444) (end 46.6852 52.9082) (width 0.5) (layer B.Cu) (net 2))
 (segment (start 46.6852 52.9082) (end 46.6852 68.707) (width 0.5) (layer B.Cu) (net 2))
 (segment (start 46.6852 68.707) (end 50.7492 72.771) (width 0.5) (layer B.Cu) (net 2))
 (segment (start 57.1246 74.7522) (end 57.1246 73.0123) (width 0.5) (layer B.Cu) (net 2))
 (segment (start 57.1246 73.0123) (end 57.4675 72.6694) (width 0.5) (layer B.Cu) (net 2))
 (segment (start 65.3034 70.358) (end 70.739 70.358) (width 0.5) (layer B.Cu) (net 11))
 (segment (start 70.5866 69.9516) (end 70.6882 50.0126) (width 0.5) (layer F.Cu) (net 11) (status 20))
 (segment (start 70.866 70.231) (end 70.5866 69.9516) (width 0.5) (layer F.Cu) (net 11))
 (via (at 70.866 70.231) (size 0.889) (layers F.Cu B.Cu) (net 11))
 (segment (start 70.739 70.358) (end 70.866 70.231) (width 0.5) (layer B.Cu) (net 11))
 (segment (start 52.9844 59.6646) (end 53.1114 59.6646) (width 0.5) (layer B.Cu) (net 15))
 (segment (start 55.118 57.658) (end 57.6834 57.658) (width 0.5) (layer B.Cu) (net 15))
 (segment (start 53.1114 59.6646) (end 55.118 57.658) (width 0.5) (layer B.Cu) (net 15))
 (segment (start 51.6382 51.9684) (end 51.6382 55.8292) (width 0.5) (layer B.Cu) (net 15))
 (segment (start 51.6382 55.8292) (end 52.9844 59.6646) (width 0.5) (layer B.Cu) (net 15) (status 20))
 (segment (start 50.3174 54.9148) (end 50.3174 57.912) (width 0.5) (layer B.Cu) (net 14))
 (segment (start 51.181 62.9412) (end 52.9844 64.7446) (width 0.5) (layer B.Cu) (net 14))
 (segment (start 51.181 58.7756) (end 51.181 62.9412) (width 0.5) (layer B.Cu) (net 14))
 (segment (start 50.3174 57.912) (end 51.181 58.7756) (width 0.5) (layer B.Cu) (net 14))
 (segment (start 52.9844 64.7446) (end 52.9844 63.3984) (width 0.5) (layer B.Cu) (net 14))
 (segment (start 56.1848 60.198) (end 57.6834 60.198) (width 0.5) (layer B.Cu) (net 14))
 (segment (start 52.9844 63.3984) (end 56.1848 60.198) (width 0.5) (layer B.Cu) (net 14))
 (segment (start 70.6882 39.8526) (end 70.6882 36.3982) (width 0.5) (layer B.Cu) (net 12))
 (segment (start 70.6882 36.3982) (end 70.8914 36.195) (width 0.5) (layer B.Cu) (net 12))
 (segment (start 65.3034 65.278) (end 73.5838 65.278) (width 0.5) (layer B.Cu) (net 6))
 (segment (start 73.5838 65.278) (end 73.6092 65.2526) (width 0.5) (layer B.Cu) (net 6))
 (segment (start 65.3034 62.738) (end 73.5838 62.738) (width 0.5) (layer B.Cu) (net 7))
 (segment (start 73.5838 62.738) (end 73.6092 62.7126) (width 0.5) (layer B.Cu) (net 7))
 (segment (start 48.26 64.2366) (end 48.26 56.6166) (width 0.5) (layer B.Cu) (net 5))
 (segment (start 57.6834 65.278) (end 56.3118 65.278) (width 0.5) (layer B.Cu) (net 5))
 (segment (start 51.7906 66.7258) (end 48.26 64.2366) (width 0.5) (layer B.Cu) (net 5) (status 20))
 (segment (start 54.864 66.7258) (end 51.7906 66.7258) (width 0.5) (layer B.Cu) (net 5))
 (segment (start 56.3118 65.278) (end 54.864 66.7258) (width 0.5) (layer B.Cu) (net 5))
 (segment (start 55.0164 70.3072) (end 55.1942 70.3072) (width 0.5) (layer B.Cu) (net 13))
 (segment (start 55.1942 70.3072) (end 57.6834 67.818) (width 0.5) (layer B.Cu) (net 13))
 (segment (start 59.2328 33.782) (end 59.2328 34.7726) (width 0.5) (layer B.Cu) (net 1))
 (segment (start 59.9694 35.5092) (end 59.9694 51.308) (width 0.5) (layer B.Cu) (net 1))
 (segment (start 59.2328 34.7726) (end 59.9694 35.5092) (width 0.5) (layer B.Cu) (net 1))
 (segment (start 59.9694 57.6834) (end 59.9694 57.5564) (width 0.5) (layer B.Cu) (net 1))
 (via (at 59.9694 57.5564) (size 0.889) (layers F.Cu B.Cu) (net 1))
 (segment (start 58.6994 52.578) (end 57.6834 52.578) (width 0.5) (layer B.Cu) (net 1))
 (segment (start 59.9694 51.308) (end 58.6994 52.578) (width 0.5) (layer B.Cu) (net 1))
 (via (at 59.9694 51.308) (size 0.889) (layers F.Cu B.Cu) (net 1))
 (segment (start 59.9694 57.5564) (end 59.9694 51.308) (width 0.5) (layer F.Cu) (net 1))
 (segment (start 61.3918 55.5879) (end 61.3918 56.134) (width 0.5) (layer B.Cu) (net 1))
 (segment (start 59.9694 72.0725) (end 59.3725 72.6694) (width 0.5) (layer B.Cu) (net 1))
 (segment (start 59.9694 57.6834) (end 59.9694 72.0725) (width 0.5) (layer B.Cu) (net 1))
 (segment (start 61.3918 56.134) (end 59.9694 57.5564) (width 0.5) (layer B.Cu) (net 1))
 (segment (start 70.6882 74.422) (end 59.9948 74.422) (width 0.5) (layer B.Cu) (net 1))
 (segment (start 59.9948 74.422) (end 59.6646 74.7522) (width 0.5) (layer B.Cu) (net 1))
 (segment (start 73.6092 70.3326) (end 73.6092 71.501) (width 0.5) (layer B.Cu) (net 1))
 (segment (start 73.6092 71.501) (end 70.6882 74.422) (width 0.5) (layer B.Cu) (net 1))
 (segment (start 65.3034 57.658) (end 63.4619 57.658) (width 0.5) (layer B.Cu) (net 1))
 (segment (start 63.4619 57.658) (end 61.3918 55.5879) (width 0.5) (layer B.Cu) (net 1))
 (segment (start 59.6646 74.7522) (end 59.6646 72.9615) (width 0.5) (layer B.Cu) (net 1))
 (segment (start 59.6646 72.9615) (end 59.3725 72.6694) (width 0.5) (layer B.Cu) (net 1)))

